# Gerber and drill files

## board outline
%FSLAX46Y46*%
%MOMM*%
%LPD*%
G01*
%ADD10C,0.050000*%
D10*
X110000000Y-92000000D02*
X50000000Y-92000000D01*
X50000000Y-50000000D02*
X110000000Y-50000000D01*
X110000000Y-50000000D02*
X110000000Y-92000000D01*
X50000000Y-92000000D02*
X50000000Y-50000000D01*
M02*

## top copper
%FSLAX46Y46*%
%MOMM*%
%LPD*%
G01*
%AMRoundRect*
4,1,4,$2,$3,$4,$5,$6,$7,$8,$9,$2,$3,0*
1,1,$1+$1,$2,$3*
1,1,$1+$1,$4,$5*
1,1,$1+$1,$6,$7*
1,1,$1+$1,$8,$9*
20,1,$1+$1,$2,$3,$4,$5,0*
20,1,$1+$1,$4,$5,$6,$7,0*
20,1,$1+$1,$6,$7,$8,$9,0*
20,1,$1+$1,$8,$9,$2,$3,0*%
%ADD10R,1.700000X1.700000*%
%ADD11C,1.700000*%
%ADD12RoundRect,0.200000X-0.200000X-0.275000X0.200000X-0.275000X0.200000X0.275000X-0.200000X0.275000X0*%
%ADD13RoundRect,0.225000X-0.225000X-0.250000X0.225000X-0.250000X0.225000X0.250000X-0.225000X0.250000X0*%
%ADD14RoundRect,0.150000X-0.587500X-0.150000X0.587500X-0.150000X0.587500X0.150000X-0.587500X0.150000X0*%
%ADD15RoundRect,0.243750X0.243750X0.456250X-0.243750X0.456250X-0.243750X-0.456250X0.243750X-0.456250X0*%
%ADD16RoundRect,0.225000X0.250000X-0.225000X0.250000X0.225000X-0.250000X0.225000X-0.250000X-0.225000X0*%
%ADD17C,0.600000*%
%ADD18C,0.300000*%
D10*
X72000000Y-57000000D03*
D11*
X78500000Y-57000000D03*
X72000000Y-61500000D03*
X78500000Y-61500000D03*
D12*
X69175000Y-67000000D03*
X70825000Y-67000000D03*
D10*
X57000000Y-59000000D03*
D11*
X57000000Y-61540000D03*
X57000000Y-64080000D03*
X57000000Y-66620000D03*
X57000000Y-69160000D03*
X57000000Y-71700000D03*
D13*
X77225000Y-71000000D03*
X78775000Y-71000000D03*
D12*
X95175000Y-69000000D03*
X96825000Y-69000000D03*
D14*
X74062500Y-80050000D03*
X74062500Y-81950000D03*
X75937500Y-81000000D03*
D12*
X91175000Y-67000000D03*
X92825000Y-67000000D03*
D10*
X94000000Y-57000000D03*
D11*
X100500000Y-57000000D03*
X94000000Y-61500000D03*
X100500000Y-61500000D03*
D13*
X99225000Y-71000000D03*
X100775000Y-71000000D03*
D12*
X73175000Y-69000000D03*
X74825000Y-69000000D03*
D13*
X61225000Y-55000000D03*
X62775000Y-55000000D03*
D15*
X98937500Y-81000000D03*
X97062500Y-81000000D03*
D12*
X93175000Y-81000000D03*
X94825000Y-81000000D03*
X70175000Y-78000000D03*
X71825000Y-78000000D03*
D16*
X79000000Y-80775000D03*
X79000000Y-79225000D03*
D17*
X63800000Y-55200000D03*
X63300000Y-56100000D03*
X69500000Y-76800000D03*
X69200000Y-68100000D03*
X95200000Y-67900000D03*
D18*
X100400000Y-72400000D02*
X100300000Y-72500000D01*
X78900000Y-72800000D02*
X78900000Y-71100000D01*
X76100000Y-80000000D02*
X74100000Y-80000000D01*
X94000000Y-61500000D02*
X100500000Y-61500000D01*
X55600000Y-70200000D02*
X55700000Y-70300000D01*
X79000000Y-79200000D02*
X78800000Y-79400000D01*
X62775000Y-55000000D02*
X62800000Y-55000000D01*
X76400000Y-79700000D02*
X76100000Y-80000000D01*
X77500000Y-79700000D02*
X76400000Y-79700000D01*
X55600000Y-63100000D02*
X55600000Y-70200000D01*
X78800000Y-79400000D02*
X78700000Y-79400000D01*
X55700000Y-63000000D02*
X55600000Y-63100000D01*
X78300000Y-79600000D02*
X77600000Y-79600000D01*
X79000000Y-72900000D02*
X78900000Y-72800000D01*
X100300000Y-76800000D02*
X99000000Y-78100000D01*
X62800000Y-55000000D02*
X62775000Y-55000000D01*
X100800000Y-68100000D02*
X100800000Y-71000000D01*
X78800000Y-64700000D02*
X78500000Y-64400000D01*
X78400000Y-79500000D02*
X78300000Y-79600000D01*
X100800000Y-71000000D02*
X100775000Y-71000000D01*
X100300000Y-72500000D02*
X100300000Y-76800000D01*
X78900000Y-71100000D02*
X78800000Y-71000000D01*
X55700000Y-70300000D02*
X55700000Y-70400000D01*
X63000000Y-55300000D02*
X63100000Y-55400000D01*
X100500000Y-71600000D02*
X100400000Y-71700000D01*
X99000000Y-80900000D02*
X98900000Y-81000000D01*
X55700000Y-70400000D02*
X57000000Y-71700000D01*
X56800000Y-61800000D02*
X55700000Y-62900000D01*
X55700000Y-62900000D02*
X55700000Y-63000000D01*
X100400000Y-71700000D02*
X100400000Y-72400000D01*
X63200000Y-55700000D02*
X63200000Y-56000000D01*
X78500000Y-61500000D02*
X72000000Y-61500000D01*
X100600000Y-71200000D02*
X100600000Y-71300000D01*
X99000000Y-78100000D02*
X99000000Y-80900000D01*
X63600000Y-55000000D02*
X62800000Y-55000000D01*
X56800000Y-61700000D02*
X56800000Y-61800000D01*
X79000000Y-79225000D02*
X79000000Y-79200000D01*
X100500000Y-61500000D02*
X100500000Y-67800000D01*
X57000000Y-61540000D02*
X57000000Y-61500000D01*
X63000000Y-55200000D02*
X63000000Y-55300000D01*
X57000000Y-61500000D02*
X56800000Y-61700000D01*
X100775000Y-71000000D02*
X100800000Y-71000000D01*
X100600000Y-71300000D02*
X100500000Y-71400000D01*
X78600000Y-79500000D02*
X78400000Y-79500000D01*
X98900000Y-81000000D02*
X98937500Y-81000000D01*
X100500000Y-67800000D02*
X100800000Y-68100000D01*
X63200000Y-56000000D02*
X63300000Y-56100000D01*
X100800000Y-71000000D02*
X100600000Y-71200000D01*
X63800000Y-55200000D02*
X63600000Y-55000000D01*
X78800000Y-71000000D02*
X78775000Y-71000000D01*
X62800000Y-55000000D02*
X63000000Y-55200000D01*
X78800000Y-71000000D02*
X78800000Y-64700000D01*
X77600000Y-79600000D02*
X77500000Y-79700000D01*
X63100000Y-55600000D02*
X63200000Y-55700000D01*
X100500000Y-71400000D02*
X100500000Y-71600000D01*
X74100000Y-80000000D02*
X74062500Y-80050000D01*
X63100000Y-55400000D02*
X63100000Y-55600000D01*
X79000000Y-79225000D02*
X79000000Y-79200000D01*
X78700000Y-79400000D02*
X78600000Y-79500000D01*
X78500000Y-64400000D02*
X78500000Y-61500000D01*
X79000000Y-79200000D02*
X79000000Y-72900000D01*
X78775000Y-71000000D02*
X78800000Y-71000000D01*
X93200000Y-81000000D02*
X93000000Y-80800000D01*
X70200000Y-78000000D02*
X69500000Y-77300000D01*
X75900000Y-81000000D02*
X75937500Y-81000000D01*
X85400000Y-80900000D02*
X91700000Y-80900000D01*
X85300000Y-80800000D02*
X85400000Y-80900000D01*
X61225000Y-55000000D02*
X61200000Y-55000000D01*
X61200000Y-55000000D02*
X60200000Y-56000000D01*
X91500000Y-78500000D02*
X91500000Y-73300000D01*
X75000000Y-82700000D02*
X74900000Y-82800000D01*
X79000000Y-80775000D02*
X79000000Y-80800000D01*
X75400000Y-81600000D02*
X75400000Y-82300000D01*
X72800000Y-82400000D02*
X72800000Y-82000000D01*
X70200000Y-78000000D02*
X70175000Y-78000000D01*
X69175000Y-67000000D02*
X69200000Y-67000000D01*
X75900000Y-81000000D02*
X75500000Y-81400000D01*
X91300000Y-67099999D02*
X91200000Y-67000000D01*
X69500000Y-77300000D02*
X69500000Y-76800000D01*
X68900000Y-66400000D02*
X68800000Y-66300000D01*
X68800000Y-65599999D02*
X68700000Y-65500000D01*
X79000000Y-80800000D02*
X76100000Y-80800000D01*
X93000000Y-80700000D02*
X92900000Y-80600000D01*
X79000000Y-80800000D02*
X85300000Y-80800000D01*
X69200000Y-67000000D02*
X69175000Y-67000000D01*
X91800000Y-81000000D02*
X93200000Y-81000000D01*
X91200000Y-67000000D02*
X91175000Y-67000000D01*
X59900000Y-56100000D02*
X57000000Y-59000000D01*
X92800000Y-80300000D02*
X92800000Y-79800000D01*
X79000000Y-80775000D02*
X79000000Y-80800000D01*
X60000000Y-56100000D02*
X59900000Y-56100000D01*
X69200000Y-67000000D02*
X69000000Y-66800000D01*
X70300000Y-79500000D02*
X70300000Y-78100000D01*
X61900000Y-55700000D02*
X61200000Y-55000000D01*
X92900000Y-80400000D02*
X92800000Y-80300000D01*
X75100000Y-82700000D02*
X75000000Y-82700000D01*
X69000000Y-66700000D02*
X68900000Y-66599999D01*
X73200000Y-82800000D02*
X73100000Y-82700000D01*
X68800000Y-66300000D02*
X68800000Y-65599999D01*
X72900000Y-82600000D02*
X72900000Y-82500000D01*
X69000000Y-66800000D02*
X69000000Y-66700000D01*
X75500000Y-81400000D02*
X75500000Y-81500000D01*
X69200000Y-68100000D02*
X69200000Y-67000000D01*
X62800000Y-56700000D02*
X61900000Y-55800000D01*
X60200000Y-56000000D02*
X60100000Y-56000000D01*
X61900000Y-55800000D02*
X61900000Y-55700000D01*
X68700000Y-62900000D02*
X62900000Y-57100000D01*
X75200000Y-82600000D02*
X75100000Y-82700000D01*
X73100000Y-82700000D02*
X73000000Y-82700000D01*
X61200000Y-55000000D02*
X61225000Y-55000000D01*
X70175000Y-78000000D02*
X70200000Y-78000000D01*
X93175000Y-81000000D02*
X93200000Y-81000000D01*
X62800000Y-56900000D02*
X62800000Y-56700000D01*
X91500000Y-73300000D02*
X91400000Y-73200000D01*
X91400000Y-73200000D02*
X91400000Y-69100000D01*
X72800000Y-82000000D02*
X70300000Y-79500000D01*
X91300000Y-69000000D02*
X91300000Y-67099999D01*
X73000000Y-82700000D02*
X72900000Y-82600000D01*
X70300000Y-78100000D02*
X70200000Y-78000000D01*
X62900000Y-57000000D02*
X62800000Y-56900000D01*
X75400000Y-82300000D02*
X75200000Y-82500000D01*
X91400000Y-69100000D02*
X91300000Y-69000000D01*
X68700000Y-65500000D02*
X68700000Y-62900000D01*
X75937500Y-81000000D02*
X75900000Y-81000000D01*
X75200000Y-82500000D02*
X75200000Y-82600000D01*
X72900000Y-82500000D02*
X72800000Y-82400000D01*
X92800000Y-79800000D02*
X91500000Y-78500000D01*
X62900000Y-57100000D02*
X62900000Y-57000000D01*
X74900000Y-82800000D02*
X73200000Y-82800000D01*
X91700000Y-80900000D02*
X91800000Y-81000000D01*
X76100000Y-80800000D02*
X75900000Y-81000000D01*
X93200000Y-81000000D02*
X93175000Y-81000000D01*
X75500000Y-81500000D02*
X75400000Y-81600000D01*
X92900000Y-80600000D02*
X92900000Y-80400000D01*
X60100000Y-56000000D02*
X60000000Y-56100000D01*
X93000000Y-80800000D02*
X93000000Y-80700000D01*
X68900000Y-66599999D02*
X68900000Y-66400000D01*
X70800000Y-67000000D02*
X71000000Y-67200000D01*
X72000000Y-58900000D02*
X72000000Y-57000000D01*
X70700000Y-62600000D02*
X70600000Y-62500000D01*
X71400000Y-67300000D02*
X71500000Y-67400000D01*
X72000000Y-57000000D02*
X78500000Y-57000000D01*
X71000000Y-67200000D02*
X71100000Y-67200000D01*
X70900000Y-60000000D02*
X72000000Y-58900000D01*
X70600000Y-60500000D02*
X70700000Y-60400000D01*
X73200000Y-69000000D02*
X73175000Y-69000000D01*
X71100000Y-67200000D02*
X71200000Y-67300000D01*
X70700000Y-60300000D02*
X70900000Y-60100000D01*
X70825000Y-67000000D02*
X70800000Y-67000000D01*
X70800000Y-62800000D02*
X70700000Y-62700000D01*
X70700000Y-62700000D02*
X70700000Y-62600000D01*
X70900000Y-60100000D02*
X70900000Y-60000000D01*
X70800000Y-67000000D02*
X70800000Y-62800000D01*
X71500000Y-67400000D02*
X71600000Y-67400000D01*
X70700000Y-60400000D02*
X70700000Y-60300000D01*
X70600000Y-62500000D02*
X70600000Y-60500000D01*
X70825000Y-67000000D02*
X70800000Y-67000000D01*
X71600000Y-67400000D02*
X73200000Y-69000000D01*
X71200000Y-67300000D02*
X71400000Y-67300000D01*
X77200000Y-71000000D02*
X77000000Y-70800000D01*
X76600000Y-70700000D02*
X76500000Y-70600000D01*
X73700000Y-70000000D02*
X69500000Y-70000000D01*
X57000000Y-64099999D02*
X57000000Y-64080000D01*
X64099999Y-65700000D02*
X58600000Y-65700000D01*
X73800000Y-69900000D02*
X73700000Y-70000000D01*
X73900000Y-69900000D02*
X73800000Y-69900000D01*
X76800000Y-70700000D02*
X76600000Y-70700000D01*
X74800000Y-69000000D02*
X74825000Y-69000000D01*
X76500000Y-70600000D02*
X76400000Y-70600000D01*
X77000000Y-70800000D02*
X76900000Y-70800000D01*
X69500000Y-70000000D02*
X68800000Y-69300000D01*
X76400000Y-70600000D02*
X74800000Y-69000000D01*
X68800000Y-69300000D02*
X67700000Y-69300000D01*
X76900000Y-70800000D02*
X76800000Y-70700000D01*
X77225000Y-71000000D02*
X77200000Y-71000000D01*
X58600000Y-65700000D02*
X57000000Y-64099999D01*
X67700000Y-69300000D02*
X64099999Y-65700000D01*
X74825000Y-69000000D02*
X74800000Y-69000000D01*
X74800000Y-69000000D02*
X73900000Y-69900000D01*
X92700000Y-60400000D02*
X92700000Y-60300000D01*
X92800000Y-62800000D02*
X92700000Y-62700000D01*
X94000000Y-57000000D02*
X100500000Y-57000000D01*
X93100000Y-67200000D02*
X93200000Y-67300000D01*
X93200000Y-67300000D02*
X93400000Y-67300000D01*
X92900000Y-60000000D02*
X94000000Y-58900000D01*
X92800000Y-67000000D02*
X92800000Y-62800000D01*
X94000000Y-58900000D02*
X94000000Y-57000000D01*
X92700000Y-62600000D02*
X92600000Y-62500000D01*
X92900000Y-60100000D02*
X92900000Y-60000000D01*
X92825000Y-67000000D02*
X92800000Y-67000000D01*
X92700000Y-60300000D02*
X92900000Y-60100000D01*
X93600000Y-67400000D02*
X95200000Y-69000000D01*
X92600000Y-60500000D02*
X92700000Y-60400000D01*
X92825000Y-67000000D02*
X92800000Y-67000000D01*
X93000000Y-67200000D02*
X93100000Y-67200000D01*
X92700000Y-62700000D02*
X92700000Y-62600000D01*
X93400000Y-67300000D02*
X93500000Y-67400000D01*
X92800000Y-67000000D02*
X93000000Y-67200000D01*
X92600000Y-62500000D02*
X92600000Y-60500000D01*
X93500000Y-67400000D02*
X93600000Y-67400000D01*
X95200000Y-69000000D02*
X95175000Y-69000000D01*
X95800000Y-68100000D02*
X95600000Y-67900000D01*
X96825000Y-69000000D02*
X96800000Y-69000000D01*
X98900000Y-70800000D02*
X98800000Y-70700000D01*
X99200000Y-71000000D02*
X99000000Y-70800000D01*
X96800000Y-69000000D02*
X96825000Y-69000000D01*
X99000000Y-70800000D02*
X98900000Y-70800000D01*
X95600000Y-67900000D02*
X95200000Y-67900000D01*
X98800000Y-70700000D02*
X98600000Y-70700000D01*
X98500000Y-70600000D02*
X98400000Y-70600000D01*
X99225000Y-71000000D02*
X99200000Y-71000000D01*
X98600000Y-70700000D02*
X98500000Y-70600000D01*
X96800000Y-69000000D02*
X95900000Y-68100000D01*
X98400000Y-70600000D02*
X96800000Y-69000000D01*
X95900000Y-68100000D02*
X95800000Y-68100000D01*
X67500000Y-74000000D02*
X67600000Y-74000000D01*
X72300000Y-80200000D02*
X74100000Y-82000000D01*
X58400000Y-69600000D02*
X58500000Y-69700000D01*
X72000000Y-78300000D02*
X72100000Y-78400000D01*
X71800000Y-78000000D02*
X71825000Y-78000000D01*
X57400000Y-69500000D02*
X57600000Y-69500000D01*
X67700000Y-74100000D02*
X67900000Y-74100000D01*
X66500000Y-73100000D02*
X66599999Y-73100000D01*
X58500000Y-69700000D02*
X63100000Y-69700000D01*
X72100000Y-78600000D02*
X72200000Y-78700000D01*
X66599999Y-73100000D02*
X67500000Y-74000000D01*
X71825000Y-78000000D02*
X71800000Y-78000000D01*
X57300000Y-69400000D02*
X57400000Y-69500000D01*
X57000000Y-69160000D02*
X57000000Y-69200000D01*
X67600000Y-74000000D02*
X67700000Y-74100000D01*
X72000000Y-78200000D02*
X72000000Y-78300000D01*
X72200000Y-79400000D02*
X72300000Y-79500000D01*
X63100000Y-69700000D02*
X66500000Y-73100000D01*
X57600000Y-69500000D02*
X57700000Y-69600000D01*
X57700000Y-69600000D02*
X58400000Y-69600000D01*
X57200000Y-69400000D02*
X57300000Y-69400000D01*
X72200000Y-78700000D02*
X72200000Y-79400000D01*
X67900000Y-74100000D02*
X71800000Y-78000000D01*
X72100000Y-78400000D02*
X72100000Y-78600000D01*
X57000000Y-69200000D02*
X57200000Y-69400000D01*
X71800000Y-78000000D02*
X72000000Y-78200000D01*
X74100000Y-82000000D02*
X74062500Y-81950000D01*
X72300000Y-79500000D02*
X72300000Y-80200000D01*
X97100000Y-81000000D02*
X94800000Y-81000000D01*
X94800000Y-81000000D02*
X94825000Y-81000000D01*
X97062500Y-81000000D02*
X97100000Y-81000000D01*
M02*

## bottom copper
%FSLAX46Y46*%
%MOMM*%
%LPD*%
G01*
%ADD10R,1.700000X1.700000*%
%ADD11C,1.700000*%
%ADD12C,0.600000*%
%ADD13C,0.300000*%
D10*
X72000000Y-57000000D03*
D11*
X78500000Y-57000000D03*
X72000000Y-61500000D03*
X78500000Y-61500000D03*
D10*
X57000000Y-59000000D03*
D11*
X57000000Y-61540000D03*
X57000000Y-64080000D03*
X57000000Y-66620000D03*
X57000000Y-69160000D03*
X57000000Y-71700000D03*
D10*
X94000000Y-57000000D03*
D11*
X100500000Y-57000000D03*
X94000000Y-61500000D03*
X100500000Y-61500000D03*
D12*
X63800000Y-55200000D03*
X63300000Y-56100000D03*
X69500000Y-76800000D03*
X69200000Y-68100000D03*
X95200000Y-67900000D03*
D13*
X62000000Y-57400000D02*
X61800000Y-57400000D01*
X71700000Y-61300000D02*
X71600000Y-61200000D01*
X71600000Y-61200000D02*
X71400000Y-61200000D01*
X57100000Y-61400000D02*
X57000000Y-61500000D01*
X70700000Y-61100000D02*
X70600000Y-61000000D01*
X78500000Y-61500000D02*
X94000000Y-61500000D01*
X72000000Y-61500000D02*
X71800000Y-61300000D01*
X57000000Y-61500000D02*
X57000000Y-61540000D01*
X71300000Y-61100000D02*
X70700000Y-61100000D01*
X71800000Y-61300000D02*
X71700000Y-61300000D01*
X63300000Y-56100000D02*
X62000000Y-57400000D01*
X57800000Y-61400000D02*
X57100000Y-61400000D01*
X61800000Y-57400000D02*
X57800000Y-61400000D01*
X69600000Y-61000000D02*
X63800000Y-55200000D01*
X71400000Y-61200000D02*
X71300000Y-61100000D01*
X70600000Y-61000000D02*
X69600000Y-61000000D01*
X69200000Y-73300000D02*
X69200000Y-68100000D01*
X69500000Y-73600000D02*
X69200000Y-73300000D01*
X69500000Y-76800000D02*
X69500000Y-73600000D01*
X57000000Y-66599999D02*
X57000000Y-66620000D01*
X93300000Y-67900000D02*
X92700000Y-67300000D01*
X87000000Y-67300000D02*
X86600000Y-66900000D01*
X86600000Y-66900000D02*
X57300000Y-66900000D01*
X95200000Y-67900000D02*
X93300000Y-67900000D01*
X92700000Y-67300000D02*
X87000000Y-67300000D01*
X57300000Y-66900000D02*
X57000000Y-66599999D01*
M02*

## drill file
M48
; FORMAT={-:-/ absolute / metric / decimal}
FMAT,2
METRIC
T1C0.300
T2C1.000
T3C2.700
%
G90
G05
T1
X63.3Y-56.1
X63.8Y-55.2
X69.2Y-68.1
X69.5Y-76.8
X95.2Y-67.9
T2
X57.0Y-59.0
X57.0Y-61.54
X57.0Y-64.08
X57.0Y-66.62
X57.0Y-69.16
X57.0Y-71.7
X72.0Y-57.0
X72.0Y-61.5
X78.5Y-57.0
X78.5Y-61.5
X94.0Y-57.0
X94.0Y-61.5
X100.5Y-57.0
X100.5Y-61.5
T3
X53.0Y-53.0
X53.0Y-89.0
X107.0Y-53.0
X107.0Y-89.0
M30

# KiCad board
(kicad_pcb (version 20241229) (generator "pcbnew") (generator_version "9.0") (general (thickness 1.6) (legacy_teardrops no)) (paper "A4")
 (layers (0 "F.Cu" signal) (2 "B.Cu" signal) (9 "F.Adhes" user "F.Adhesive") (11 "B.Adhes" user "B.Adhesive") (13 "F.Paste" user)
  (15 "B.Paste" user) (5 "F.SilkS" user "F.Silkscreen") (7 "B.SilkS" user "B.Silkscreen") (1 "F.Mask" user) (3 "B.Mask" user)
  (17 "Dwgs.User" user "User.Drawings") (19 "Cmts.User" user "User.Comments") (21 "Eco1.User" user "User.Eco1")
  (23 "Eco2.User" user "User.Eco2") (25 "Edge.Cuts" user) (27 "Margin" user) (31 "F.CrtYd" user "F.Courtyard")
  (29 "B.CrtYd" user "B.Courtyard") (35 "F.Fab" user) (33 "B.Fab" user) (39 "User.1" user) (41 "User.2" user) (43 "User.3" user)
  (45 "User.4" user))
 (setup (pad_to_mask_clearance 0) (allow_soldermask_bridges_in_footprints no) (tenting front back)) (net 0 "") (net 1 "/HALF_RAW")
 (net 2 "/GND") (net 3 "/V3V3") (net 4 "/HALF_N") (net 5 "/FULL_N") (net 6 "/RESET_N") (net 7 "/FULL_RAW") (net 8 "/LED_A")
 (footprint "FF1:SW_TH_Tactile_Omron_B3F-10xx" (layer "F.Cu") (at 72 57)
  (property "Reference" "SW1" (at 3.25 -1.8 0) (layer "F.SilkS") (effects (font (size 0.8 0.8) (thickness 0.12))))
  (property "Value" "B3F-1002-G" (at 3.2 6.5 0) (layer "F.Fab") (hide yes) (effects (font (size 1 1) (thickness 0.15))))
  (pad "1" thru_hole rect (at 0 0) (size 1.7 1.7) (drill 1) (layers "*.Cu" "*.Mask") (remove_unused_layers no) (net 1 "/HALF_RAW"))
  (pad "1" thru_hole circle (at 6.5 0) (size 1.7 1.7) (drill 1) (layers "*.Cu" "*.Mask") (remove_unused_layers no) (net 1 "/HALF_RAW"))
  (pad "2" thru_hole circle (at 0 4.5) (size 1.7 1.7) (drill 1) (layers "*.Cu" "*.Mask") (remove_unused_layers no) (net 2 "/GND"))
  (pad "2" thru_hole circle (at 6.5 4.5) (size 1.7 1.7) (drill 1) (layers "*.Cu" "*.Mask") (remove_unused_layers no) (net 2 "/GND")))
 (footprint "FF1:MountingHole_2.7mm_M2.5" (layer "F.Cu") (at 53 53)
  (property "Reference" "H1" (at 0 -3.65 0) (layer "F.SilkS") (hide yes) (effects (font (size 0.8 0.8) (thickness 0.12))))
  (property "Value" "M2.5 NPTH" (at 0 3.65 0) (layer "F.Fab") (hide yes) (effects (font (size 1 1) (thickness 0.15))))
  (pad "" np_thru_hole circle (at 0 0) (size 2.7 2.7) (drill 2.7) (layers "*.Cu" "*.Mask")))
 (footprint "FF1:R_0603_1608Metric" (layer "F.Cu") (at 70 67)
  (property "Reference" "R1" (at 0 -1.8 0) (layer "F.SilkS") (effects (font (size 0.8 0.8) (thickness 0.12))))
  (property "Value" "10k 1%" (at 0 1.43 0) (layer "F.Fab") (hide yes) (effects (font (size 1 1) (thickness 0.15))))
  (pad "1" smd roundrect (at -0.825 0) (size 0.8 0.95) (layers "F.Cu" "F.Mask" "F.Paste") (roundrect_rratio 0.25) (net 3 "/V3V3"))
  (pad "2" smd roundrect (at 0.825 0) (size 0.8 0.95) (layers "F.Cu" "F.Mask" "F.Paste") (roundrect_rratio 0.25) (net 1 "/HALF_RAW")))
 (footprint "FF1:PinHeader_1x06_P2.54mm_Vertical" (layer "F.Cu") (at 57 59)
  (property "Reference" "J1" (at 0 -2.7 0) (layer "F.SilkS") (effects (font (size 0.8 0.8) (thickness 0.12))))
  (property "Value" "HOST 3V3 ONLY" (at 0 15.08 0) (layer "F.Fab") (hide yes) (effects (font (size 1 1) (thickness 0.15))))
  (pad "1" thru_hole rect (at 0 0) (size 1.7 1.7) (drill 1) (layers "*.Cu" "*.Mask") (remove_unused_layers no) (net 3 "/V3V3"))
  (pad "2" thru_hole circle (at 0 2.54) (size 1.7 1.7) (drill 1) (layers "*.Cu" "*.Mask") (remove_unused_layers no) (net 2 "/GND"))
  (pad "3" thru_hole circle (at 0 5.08) (size 1.7 1.7) (drill 1) (layers "*.Cu" "*.Mask") (remove_unused_layers no) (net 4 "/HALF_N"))
  (pad "4" thru_hole circle (at 0 7.62) (size 1.7 1.7) (drill 1) (layers "*.Cu" "*.Mask") (remove_unused_layers no) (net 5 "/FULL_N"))
  (pad "5" thru_hole circle (at 0 10.16) (size 1.7 1.7) (drill 1) (layers "*.Cu" "*.Mask") (remove_unused_layers no) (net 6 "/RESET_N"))
  (pad "6" thru_hole circle (at 0 12.7) (size 1.7 1.7) (drill 1) (layers "*.Cu" "*.Mask") (remove_unused_layers no) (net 2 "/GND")))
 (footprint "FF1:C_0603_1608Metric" (layer "F.Cu") (at 78 71)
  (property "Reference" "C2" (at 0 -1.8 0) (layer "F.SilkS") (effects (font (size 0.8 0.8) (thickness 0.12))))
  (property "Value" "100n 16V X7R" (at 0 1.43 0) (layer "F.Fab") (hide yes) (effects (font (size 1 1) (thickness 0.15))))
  (pad "1" smd roundrect (at -0.775 0) (size 0.9 0.95) (layers "F.Cu" "F.Mask" "F.Paste") (roundrect_rratio 0.25) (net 4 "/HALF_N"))
  (pad "2" smd roundrect (at 0.775 0) (size 0.9 0.95) (layers "F.Cu" "F.Mask" "F.Paste") (roundrect_rratio 0.25) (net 2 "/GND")))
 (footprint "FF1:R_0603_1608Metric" (layer "F.Cu") (at 96 69)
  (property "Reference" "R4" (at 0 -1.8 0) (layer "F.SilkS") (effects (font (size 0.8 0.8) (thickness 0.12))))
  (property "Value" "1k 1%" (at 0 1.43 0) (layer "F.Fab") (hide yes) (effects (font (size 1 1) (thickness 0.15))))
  (pad "1" smd roundrect (at -0.825 0) (size 0.8 0.95) (layers "F.Cu" "F.Mask" "F.Paste") (roundrect_rratio 0.25) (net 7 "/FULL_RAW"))
  (pad "2" smd roundrect (at 0.825 0) (size 0.8 0.95) (layers "F.Cu" "F.Mask" "F.Paste") (roundrect_rratio 0.25) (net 5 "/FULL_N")))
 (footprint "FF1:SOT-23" (layer "F.Cu") (at 75 81)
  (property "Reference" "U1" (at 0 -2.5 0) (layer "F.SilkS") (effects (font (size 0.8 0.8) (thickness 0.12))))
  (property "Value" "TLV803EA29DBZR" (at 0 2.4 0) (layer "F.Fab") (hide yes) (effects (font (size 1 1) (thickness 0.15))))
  (pad "1" smd roundrect (at -0.9375 -0.95) (size 1.475 0.6) (layers "F.Cu" "F.Mask" "F.Paste") (roundrect_rratio 0.25) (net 2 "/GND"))
  (pad "2" smd roundrect (at -0.9375 0.95) (size 1.475 0.6) (layers "F.Cu" "F.Mask" "F.Paste") (roundrect_rratio 0.25) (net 6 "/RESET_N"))
  (pad "3" smd roundrect (at 0.9375 0) (size 1.475 0.6) (layers "F.Cu" "F.Mask" "F.Paste") (roundrect_rratio 0.25) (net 3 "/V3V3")))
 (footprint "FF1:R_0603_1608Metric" (layer "F.Cu") (at 92 67)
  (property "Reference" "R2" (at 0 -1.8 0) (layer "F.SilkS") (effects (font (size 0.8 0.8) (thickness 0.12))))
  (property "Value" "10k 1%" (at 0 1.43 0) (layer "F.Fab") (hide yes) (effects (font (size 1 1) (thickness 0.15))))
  (pad "1" smd roundrect (at -0.825 0) (size 0.8 0.95) (layers "F.Cu" "F.Mask" "F.Paste") (roundrect_rratio 0.25) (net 3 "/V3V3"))
  (pad "2" smd roundrect (at 0.825 0) (size 0.8 0.95) (layers "F.Cu" "F.Mask" "F.Paste") (roundrect_rratio 0.25) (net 7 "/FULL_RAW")))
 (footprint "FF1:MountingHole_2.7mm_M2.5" (layer "F.Cu") (at 107 53)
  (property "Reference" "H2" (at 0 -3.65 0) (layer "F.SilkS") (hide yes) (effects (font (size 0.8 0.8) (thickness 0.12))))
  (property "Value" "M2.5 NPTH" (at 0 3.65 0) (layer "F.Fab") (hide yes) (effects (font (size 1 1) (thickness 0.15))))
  (pad "" np_thru_hole circle (at 0 0) (size 2.7 2.7) (drill 2.7) (layers "*.Cu" "*.Mask")))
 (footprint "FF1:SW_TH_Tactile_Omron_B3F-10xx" (layer "F.Cu") (at 94 57)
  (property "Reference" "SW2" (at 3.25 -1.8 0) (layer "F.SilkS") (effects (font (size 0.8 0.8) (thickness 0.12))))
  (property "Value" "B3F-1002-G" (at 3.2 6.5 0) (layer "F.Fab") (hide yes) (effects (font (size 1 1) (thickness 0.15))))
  (pad "1" thru_hole rect (at 0 0) (size 1.7 1.7) (drill 1) (layers "*.Cu" "*.Mask") (remove_unused_layers no) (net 7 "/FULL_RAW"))
  (pad "1" thru_hole circle (at 6.5 0) (size 1.7 1.7) (drill 1) (layers "*.Cu" "*.Mask") (remove_unused_layers no) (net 7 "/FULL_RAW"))
  (pad "2" thru_hole circle (at 0 4.5) (size 1.7 1.7) (drill 1) (layers "*.Cu" "*.Mask") (remove_unused_layers no) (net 2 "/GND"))
  (pad "2" thru_hole circle (at 6.5 4.5) (size 1.7 1.7) (drill 1) (layers "*.Cu" "*.Mask") (remove_unused_layers no) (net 2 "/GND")))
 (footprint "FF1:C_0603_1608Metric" (layer "F.Cu") (at 100 71)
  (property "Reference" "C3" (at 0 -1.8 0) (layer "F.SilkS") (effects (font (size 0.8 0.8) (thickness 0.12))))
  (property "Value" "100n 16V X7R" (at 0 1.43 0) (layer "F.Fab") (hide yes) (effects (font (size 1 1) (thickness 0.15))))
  (pad "1" smd roundrect (at -0.775 0) (size 0.9 0.95) (layers "F.Cu" "F.Mask" "F.Paste") (roundrect_rratio 0.25) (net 5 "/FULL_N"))
  (pad "2" smd roundrect (at 0.775 0) (size 0.9 0.95) (layers "F.Cu" "F.Mask" "F.Paste") (roundrect_rratio 0.25) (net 2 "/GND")))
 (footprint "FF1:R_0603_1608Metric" (layer "F.Cu") (at 74 69)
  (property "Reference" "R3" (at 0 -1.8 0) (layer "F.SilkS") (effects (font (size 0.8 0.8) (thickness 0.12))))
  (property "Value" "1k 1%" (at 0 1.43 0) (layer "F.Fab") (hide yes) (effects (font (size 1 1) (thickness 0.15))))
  (pad "1" smd roundrect (at -0.825 0) (size 0.8 0.95) (layers "F.Cu" "F.Mask" "F.Paste") (roundrect_rratio 0.25) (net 1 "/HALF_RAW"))
  (pad "2" smd roundrect (at 0.825 0) (size 0.8 0.95) (layers "F.Cu" "F.Mask" "F.Paste") (roundrect_rratio 0.25) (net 4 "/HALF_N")))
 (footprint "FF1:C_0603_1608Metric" (layer "F.Cu") (at 62 55)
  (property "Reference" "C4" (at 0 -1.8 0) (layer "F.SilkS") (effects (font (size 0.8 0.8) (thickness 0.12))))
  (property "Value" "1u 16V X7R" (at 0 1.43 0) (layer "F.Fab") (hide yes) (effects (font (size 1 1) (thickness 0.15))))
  (pad "1" smd roundrect (at -0.775 0) (size 0.9 0.95) (layers "F.Cu" "F.Mask" "F.Paste") (roundrect_rratio 0.25) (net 3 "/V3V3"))
  (pad "2" smd roundrect (at 0.775 0) (size 0.9 0.95) (layers "F.Cu" "F.Mask" "F.Paste") (roundrect_rratio 0.25) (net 2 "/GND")))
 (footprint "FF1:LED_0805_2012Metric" (layer "F.Cu") (at 98 81 180)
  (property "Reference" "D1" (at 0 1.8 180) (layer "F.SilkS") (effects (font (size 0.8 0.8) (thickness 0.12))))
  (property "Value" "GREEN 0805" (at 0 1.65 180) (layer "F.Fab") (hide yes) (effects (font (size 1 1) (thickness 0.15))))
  (pad "1" smd roundrect (at -0.9375 0 180) (size 0.975 1.4) (layers "F.Cu" "F.Mask" "F.Paste") (roundrect_rratio 0.25) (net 2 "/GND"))
  (pad "2" smd roundrect (at 0.9375 0 180) (size 0.975 1.4) (layers "F.Cu" "F.Mask" "F.Paste") (roundrect_rratio 0.25) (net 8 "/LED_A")))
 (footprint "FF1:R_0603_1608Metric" (layer "F.Cu") (at 94 81)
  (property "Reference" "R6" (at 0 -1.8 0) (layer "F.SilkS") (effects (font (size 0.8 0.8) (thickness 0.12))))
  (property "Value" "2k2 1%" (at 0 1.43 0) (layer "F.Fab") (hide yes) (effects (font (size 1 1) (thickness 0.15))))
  (pad "1" smd roundrect (at -0.825 0) (size 0.8 0.95) (layers "F.Cu" "F.Mask" "F.Paste") (roundrect_rratio 0.25) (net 3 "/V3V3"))
  (pad "2" smd roundrect (at 0.825 0) (size 0.8 0.95) (layers "F.Cu" "F.Mask" "F.Paste") (roundrect_rratio 0.25) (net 8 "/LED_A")))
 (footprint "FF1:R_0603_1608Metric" (layer "F.Cu") (at 71 78)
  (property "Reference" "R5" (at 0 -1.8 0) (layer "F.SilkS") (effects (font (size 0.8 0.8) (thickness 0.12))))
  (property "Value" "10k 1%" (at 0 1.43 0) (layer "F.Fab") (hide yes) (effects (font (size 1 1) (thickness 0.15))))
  (pad "1" smd roundrect (at -0.825 0) (size 0.8 0.95) (layers "F.Cu" "F.Mask" "F.Paste") (roundrect_rratio 0.25) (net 3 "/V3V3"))
  (pad "2" smd roundrect (at 0.825 0) (size 0.8 0.95) (layers "F.Cu" "F.Mask" "F.Paste") (roundrect_rratio 0.25) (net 6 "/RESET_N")))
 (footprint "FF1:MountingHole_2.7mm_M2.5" (layer "F.Cu") (at 53 89)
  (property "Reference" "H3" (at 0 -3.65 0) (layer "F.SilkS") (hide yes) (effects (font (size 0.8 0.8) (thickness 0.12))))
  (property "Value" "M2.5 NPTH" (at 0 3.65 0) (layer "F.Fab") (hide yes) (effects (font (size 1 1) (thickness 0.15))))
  (pad "" np_thru_hole circle (at 0 0) (size 2.7 2.7) (drill 2.7) (layers "*.Cu" "*.Mask")))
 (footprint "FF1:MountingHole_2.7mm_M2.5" (layer "F.Cu") (at 107 89)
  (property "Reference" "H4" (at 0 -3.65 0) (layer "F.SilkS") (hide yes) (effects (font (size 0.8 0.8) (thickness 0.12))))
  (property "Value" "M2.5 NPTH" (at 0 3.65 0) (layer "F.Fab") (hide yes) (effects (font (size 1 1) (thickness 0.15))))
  (pad "" np_thru_hole circle (at 0 0) (size 2.7 2.7) (drill 2.7) (layers "*.Cu" "*.Mask")))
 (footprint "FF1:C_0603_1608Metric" (layer "F.Cu") (at 79 80 90)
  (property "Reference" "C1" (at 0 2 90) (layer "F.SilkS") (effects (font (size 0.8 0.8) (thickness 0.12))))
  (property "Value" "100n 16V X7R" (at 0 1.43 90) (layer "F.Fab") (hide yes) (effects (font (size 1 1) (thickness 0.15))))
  (pad "1" smd roundrect (at -0.775 0 90) (size 0.9 0.95) (layers "F.Cu" "F.Mask" "F.Paste") (roundrect_rratio 0.25) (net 3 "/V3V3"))
  (pad "2" smd roundrect (at 0.775 0 90) (size 0.9 0.95) (layers "F.Cu" "F.Mask" "F.Paste") (roundrect_rratio 0.25) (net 2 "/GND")))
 (gr_line (start 110 92) (end 50 92) (stroke (width 0.05) (type default)) (layer "Edge.Cuts"))
 (gr_line (start 50 50) (end 110 50) (stroke (width 0.05) (type default)) (layer "Edge.Cuts"))
 (gr_line (start 110 50) (end 110 92) (stroke (width 0.05) (type default)) (layer "Edge.Cuts"))
 (gr_line (start 50 92) (end 50 50) (stroke (width 0.05) (type default)) (layer "Edge.Cuts"))
 (segment (start 100.4 72.4) (end 100.3 72.5) (width 0.3) (layer "F.Cu") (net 2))
 (segment (start 78.9 72.8) (end 78.9 71.1) (width 0.3) (layer "F.Cu") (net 2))
 (segment (start 76.1 80) (end 74.1 80) (width 0.3) (layer "F.Cu") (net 2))
 (segment (start 94 61.5) (end 100.5 61.5) (width 0.3) (layer "F.Cu") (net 2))
 (segment (start 55.6 70.2) (end 55.7 70.3) (width 0.3) (layer "F.Cu") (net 2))
 (segment (start 79 79.2) (end 78.8 79.4) (width 0.3) (layer "F.Cu") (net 2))
 (segment (start 62.775 55) (end 62.8 55) (width 0.3) (layer "F.Cu") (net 2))
 (segment (start 76.4 79.7) (end 76.1 80) (width 0.3) (layer "F.Cu") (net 2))
 (segment (start 77.5 79.7) (end 76.4 79.7) (width 0.3) (layer "F.Cu") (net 2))
 (segment (start 55.6 63.1) (end 55.6 70.2) (width 0.3) (layer "F.Cu") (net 2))
 (segment (start 78.8 79.4) (end 78.7 79.4) (width 0.3) (layer "F.Cu") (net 2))
 (segment (start 55.7 63) (end 55.6 63.1) (width 0.3) (layer "F.Cu") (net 2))
 (segment (start 78.3 79.6) (end 77.6 79.6) (width 0.3) (layer "F.Cu") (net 2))
 (segment (start 79 72.9) (end 78.9 72.8) (width 0.3) (layer "F.Cu") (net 2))
 (segment (start 100.3 76.8) (end 99 78.1) (width 0.3) (layer "F.Cu") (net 2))
 (segment (start 62.8 55) (end 62.775 55) (width 0.3) (layer "F.Cu") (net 2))
 (segment (start 100.8 68.1) (end 100.8 71) (width 0.3) (layer "F.Cu") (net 2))
 (segment (start 78.8 64.7) (end 78.5 64.4) (width 0.3) (layer "F.Cu") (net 2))
 (segment (start 78.4 79.5) (end 78.3 79.6) (width 0.3) (layer "F.Cu") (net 2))
 (segment (start 100.8 71) (end 100.775 71) (width 0.3) (layer "F.Cu") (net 2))
 (segment (start 100.3 72.5) (end 100.3 76.8) (width 0.3) (layer "F.Cu") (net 2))
 (segment (start 78.9 71.1) (end 78.8 71) (width 0.3) (layer "F.Cu") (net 2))
 (segment (start 55.7 70.3) (end 55.7 70.4) (width 0.3) (layer "F.Cu") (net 2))
 (segment (start 63 55.3) (end 63.1 55.4) (width 0.3) (layer "F.Cu") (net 2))
 (segment (start 100.5 71.6) (end 100.4 71.7) (width 0.3) (layer "F.Cu") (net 2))
 (segment (start 99 80.9) (end 98.9 81) (width 0.3) (layer "F.Cu") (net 2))
 (segment (start 55.7 70.4) (end 57 71.7) (width 0.3) (layer "F.Cu") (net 2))
 (segment (start 56.8 61.8) (end 55.7 62.9) (width 0.3) (layer "F.Cu") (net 2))
 (segment (start 55.7 62.9) (end 55.7 63) (width 0.3) (layer "F.Cu") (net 2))
 (segment (start 100.4 71.7) (end 100.4 72.4) (width 0.3) (layer "F.Cu") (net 2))
 (segment (start 63.2 55.7) (end 63.2 56) (width 0.3) (layer "F.Cu") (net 2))
 (segment (start 78.5 61.5) (end 72 61.5) (width 0.3) (layer "F.Cu") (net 2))
 (segment (start 100.6 71.2) (end 100.6 71.3) (width 0.3) (layer "F.Cu") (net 2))
 (segment (start 99 78.1) (end 99 80.9) (width 0.3) (layer "F.Cu") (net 2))
 (segment (start 63.6 55) (end 62.8 55) (width 0.3) (layer "F.Cu") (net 2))
 (segment (start 56.8 61.7) (end 56.8 61.8) (width 0.3) (layer "F.Cu") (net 2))
 (segment (start 79 79.225) (end 79 79.2) (width 0.3) (layer "F.Cu") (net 2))
 (segment (start 100.5 61.5) (end 100.5 67.8) (width 0.3) (layer "F.Cu") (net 2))
 (segment (start 57 61.54) (end 57 61.5) (width 0.3) (layer "F.Cu") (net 2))
 (segment (start 63 55.2) (end 63 55.3) (width 0.3) (layer "F.Cu") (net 2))
 (segment (start 57 61.5) (end 56.8 61.7) (width 0.3) (layer "F.Cu") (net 2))
 (segment (start 100.775 71) (end 100.8 71) (width 0.3) (layer "F.Cu") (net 2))
 (segment (start 100.6 71.3) (end 100.5 71.4) (width 0.3) (layer "F.Cu") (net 2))
 (segment (start 78.6 79.5) (end 78.4 79.5) (width 0.3) (layer "F.Cu") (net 2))
 (segment (start 98.9 81) (end 98.9375 81) (width 0.3) (layer "F.Cu") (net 2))
 (segment (start 100.5 67.8) (end 100.8 68.1) (width 0.3) (layer "F.Cu") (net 2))
 (segment (start 63.2 56) (end 63.3 56.1) (width 0.3) (layer "F.Cu") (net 2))
 (segment (start 100.8 71) (end 100.6 71.2) (width 0.3) (layer "F.Cu") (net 2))
 (segment (start 63.8 55.2) (end 63.6 55) (width 0.3) (layer "F.Cu") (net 2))
 (segment (start 78.8 71) (end 78.775 71) (width 0.3) (layer "F.Cu") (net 2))
 (segment (start 62.8 55) (end 63 55.2) (width 0.3) (layer "F.Cu") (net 2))
 (segment (start 78.8 71) (end 78.8 64.7) (width 0.3) (layer "F.Cu") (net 2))
 (segment (start 77.6 79.6) (end 77.5 79.7) (width 0.3) (layer "F.Cu") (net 2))
 (segment (start 63.1 55.6) (end 63.2 55.7) (width 0.3) (layer "F.Cu") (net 2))
 (segment (start 100.5 71.4) (end 100.5 71.6) (width 0.3) (layer "F.Cu") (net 2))
 (segment (start 74.1 80) (end 74.0625 80.05) (width 0.3) (layer "F.Cu") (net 2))
 (segment (start 63.1 55.4) (end 63.1 55.6) (width 0.3) (layer "F.Cu") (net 2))
 (segment (start 79 79.225) (end 79 79.2) (width 0.3) (layer "F.Cu") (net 2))
 (segment (start 78.7 79.4) (end 78.6 79.5) (width 0.3) (layer "F.Cu") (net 2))
 (segment (start 78.5 64.4) (end 78.5 61.5) (width 0.3) (layer "F.Cu") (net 2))
 (segment (start 79 79.2) (end 79 72.9) (width 0.3) (layer "F.Cu") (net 2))
 (segment (start 78.775 71) (end 78.8 71) (width 0.3) (layer "F.Cu") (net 2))
 (via (at 63.8 55.2) (size 0.6) (drill 0.3) (layers "F.Cu" "B.Cu") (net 2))
 (via (at 63.3 56.1) (size 0.6) (drill 0.3) (layers "F.Cu" "B.Cu") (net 2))
 (segment (start 62 57.4) (end 61.8 57.4) (width 0.3) (layer "B.Cu") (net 2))
 (segment (start 71.7 61.3) (end 71.6 61.2) (width 0.3) (layer "B.Cu") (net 2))
 (segment (start 71.6 61.2) (end 71.4 61.2) (width 0.3) (layer "B.Cu") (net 2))
 (segment (start 57.1 61.4) (end 57 61.5) (width 0.3) (layer "B.Cu") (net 2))
 (segment (start 70.7 61.1) (end 70.6 61) (width 0.3) (layer "B.Cu") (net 2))
 (segment (start 78.5 61.5) (end 94 61.5) (width 0.3) (layer "B.Cu") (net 2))
 (segment (start 72 61.5) (end 71.8 61.3) (width 0.3) (layer "B.Cu") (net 2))
 (segment (start 57 61.5) (end 57 61.54) (width 0.3) (layer "B.Cu") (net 2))
 (segment (start 71.3 61.1) (end 70.7 61.1) (width 0.3) (layer "B.Cu") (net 2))
 (segment (start 71.8 61.3) (end 71.7 61.3) (width 0.3) (layer "B.Cu") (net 2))
 (segment (start 63.3 56.1) (end 62 57.4) (width 0.3) (layer "B.Cu") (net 2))
 (segment (start 57.8 61.4) (end 57.1 61.4) (width 0.3) (layer "B.Cu") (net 2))
 (segment (start 61.8 57.4) (end 57.8 61.4) (width 0.3) (layer "B.Cu") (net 2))
 (segment (start 69.6 61) (end 63.8 55.2) (width 0.3) (layer "B.Cu") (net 2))
 (segment (start 71.4 61.2) (end 71.3 61.1) (width 0.3) (layer "B.Cu") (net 2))
 (segment (start 70.6 61) (end 69.6 61) (width 0.3) (layer "B.Cu") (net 2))
 (segment (start 93.2 81) (end 93 80.8) (width 0.3) (layer "F.Cu") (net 3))
 (segment (start 70.2 78) (end 69.5 77.3) (width 0.3) (layer "F.Cu") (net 3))
 (segment (start 75.9 81) (end 75.9375 81) (width 0.3) (layer "F.Cu") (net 3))
 (segment (start 85.4 80.9) (end 91.7 80.9) (width 0.3) (layer "F.Cu") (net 3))
 (segment (start 85.3 80.8) (end 85.4 80.9) (width 0.3) (layer "F.Cu") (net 3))
 (segment (start 61.225 55) (end 61.2 55) (width 0.3) (layer "F.Cu") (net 3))
 (segment (start 61.2 55) (end 60.2 56) (width 0.3) (layer "F.Cu") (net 3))
 (segment (start 91.5 78.5) (end 91.5 73.3) (width 0.3) (layer "F.Cu") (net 3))
 (segment (start 75 82.7) (end 74.9 82.8) (width 0.3) (layer "F.Cu") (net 3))
 (segment (start 79 80.775) (end 79 80.8) (width 0.3) (layer "F.Cu") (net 3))
 (segment (start 75.4 81.6) (end 75.4 82.3) (width 0.3) (layer "F.Cu") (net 3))
 (segment (start 72.8 82.4) (end 72.8 82) (width 0.3) (layer "F.Cu") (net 3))
 (segment (start 70.2 78) (end 70.175 78) (width 0.3) (layer "F.Cu") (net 3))
 (segment (start 69.175 67) (end 69.2 67) (width 0.3) (layer "F.Cu") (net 3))
 (segment (start 75.9 81) (end 75.5 81.4) (width 0.3) (layer "F.Cu") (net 3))
 (segment (start 91.3 67.099999) (end 91.2 67) (width 0.3) (layer "F.Cu") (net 3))
 (segment (start 69.5 77.3) (end 69.5 76.8) (width 0.3) (layer "F.Cu") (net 3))
 (segment (start 68.9 66.4) (end 68.8 66.3) (width 0.3) (layer "F.Cu") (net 3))
 (segment (start 68.8 65.599999) (end 68.7 65.5) (width 0.3) (layer "F.Cu") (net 3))
 (segment (start 79 80.8) (end 76.1 80.8) (width 0.3) (layer "F.Cu") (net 3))
 (segment (start 93 80.7) (end 92.9 80.6) (width 0.3) (layer "F.Cu") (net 3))
 (segment (start 79 80.8) (end 85.3 80.8) (width 0.3) (layer "F.Cu") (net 3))
 (segment (start 69.2 67) (end 69.175 67) (width 0.3) (layer "F.Cu") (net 3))
 (segment (start 91.8 81) (end 93.2 81) (width 0.3) (layer "F.Cu") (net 3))
 (segment (start 91.2 67) (end 91.175 67) (width 0.3) (layer "F.Cu") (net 3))
 (segment (start 59.9 56.1) (end 57 59) (width 0.3) (layer "F.Cu") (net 3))
 (segment (start 92.8 80.3) (end 92.8 79.8) (width 0.3) (layer "F.Cu") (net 3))
 (segment (start 79 80.775) (end 79 80.8) (width 0.3) (layer "F.Cu") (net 3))
 (segment (start 60 56.1) (end 59.9 56.1) (width 0.3) (layer "F.Cu") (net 3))
 (segment (start 69.2 67) (end 69 66.8) (width 0.3) (layer "F.Cu") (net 3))
 (segment (start 70.3 79.5) (end 70.3 78.1) (width 0.3) (layer "F.Cu") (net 3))
 (segment (start 61.9 55.7) (end 61.2 55) (width 0.3) (layer "F.Cu") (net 3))
 (segment (start 92.9 80.4) (end 92.8 80.3) (width 0.3) (layer "F.Cu") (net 3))
 (segment (start 75.1 82.7) (end 75 82.7) (width 0.3) (layer "F.Cu") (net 3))
 (segment (start 69 66.7) (end 68.9 66.599999) (width 0.3) (layer "F.Cu") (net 3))
 (segment (start 73.2 82.8) (end 73.1 82.7) (width 0.3) (layer "F.Cu") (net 3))
 (segment (start 68.8 66.3) (end 68.8 65.599999) (width 0.3) (layer "F.Cu") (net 3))
 (segment (start 72.9 82.6) (end 72.9 82.5) (width 0.3) (layer "F.Cu") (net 3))
 (segment (start 69 66.8) (end 69 66.7) (width 0.3) (layer "F.Cu") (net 3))
 (segment (start 75.5 81.4) (end 75.5 81.5) (width 0.3) (layer "F.Cu") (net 3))
 (segment (start 69.2 68.1) (end 69.2 67) (width 0.3) (layer "F.Cu") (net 3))
 (segment (start 62.8 56.7) (end 61.9 55.8) (width 0.3) (layer "F.Cu") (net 3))
 (segment (start 60.2 56) (end 60.1 56) (width 0.3) (layer "F.Cu") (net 3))
 (segment (start 61.9 55.8) (end 61.9 55.7) (width 0.3) (layer "F.Cu") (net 3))
 (segment (start 68.7 62.9) (end 62.9 57.1) (width 0.3) (layer "F.Cu") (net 3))
 (segment (start 75.2 82.6) (end 75.1 82.7) (width 0.3) (layer "F.Cu") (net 3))
 (segment (start 73.1 82.7) (end 73 82.7) (width 0.3) (layer "F.Cu") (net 3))
 (segment (start 61.2 55) (end 61.225 55) (width 0.3) (layer "F.Cu") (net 3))
 (segment (start 70.175 78) (end 70.2 78) (width 0.3) (layer "F.Cu") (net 3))
 (segment (start 93.175 81) (end 93.2 81) (width 0.3) (layer "F.Cu") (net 3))
 (segment (start 62.8 56.9) (end 62.8 56.7) (width 0.3) (layer "F.Cu") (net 3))
 (segment (start 91.5 73.3) (end 91.4 73.2) (width 0.3) (layer "F.Cu") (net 3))
 (segment (start 91.4 73.2) (end 91.4 69.1) (width 0.3) (layer "F.Cu") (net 3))
 (segment (start 72.8 82) (end 70.3 79.5) (width 0.3) (layer "F.Cu") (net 3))
 (segment (start 91.3 69) (end 91.3 67.099999) (width 0.3) (layer "F.Cu") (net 3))
 (segment (start 73 82.7) (end 72.9 82.6) (width 0.3) (layer "F.Cu") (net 3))
 (segment (start 70.3 78.1) (end 70.2 78) (width 0.3) (layer "F.Cu") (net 3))
 (segment (start 62.9 57) (end 62.8 56.9) (width 0.3) (layer "F.Cu") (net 3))
 (segment (start 75.4 82.3) (end 75.2 82.5) (width 0.3) (layer "F.Cu") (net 3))
 (segment (start 91.4 69.1) (end 91.3 69) (width 0.3) (layer "F.Cu") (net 3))
 (segment (start 68.7 65.5) (end 68.7 62.9) (width 0.3) (layer "F.Cu") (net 3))
 (segment (start 75.9375 81) (end 75.9 81) (width 0.3) (layer "F.Cu") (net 3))
 (segment (start 75.2 82.5) (end 75.2 82.6) (width 0.3) (layer "F.Cu") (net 3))
 (segment (start 72.9 82.5) (end 72.8 82.4) (width 0.3) (layer "F.Cu") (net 3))
 (segment (start 92.8 79.8) (end 91.5 78.5) (width 0.3) (layer "F.Cu") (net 3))
 (segment (start 62.9 57.1) (end 62.9 57) (width 0.3) (layer "F.Cu") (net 3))
 (segment (start 74.9 82.8) (end 73.2 82.8) (width 0.3) (layer "F.Cu") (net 3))
 (segment (start 91.7 80.9) (end 91.8 81) (width 0.3) (layer "F.Cu") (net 3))
 (segment (start 76.1 80.8) (end 75.9 81) (width 0.3) (layer "F.Cu") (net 3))
 (segment (start 93.2 81) (end 93.175 81) (width 0.3) (layer "F.Cu") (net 3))
 (segment (start 75.5 81.5) (end 75.4 81.6) (width 0.3) (layer "F.Cu") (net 3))
 (segment (start 92.9 80.6) (end 92.9 80.4) (width 0.3) (layer "F.Cu") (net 3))
 (segment (start 60.1 56) (end 60 56.1) (width 0.3) (layer "F.Cu") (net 3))
 (segment (start 93 80.8) (end 93 80.7) (width 0.3) (layer "F.Cu") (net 3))
 (segment (start 68.9 66.599999) (end 68.9 66.4) (width 0.3) (layer "F.Cu") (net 3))
 (via (at 69.5 76.8) (size 0.6) (drill 0.3) (layers "F.Cu" "B.Cu") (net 3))
 (via (at 69.2 68.1) (size 0.6) (drill 0.3) (layers "F.Cu" "B.Cu") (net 3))
 (segment (start 69.2 73.3) (end 69.2 68.1) (width 0.3) (layer "B.Cu") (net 3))
 (segment (start 69.5 73.6) (end 69.2 73.3) (width 0.3) (layer "B.Cu") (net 3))
 (segment (start 69.5 76.8) (end 69.5 73.6) (width 0.3) (layer "B.Cu") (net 3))
 (segment (start 70.8 67) (end 71 67.2) (width 0.3) (layer "F.Cu") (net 1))
 (segment (start 72 58.9) (end 72 57) (width 0.3) (layer "F.Cu") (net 1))
 (segment (start 70.7 62.6) (end 70.6 62.5) (width 0.3) (layer "F.Cu") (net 1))
 (segment (start 71.4 67.3) (end 71.5 67.4) (width 0.3) (layer "F.Cu") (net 1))
 (segment (start 72 57) (end 78.5 57) (width 0.3) (layer "F.Cu") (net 1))
 (segment (start 71 67.2) (end 71.1 67.2) (width 0.3) (layer "F.Cu") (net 1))
 (segment (start 70.9 60) (end 72 58.9) (width 0.3) (layer "F.Cu") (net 1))
 (segment (start 70.6 60.5) (end 70.7 60.4) (width 0.3) (layer "F.Cu") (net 1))
 (segment (start 73.2 69) (end 73.175 69) (width 0.3) (layer "F.Cu") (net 1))
 (segment (start 71.1 67.2) (end 71.2 67.3) (width 0.3) (layer "F.Cu") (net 1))
 (segment (start 70.7 60.3) (end 70.9 60.1) (width 0.3) (layer "F.Cu") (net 1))
 (segment (start 70.825 67) (end 70.8 67) (width 0.3) (layer "F.Cu") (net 1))
 (segment (start 70.8 62.8) (end 70.7 62.7) (width 0.3) (layer "F.Cu") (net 1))
 (segment (start 70.7 62.7) (end 70.7 62.6) (width 0.3) (layer "F.Cu") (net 1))
 (segment (start 70.9 60.1) (end 70.9 60) (width 0.3) (layer "F.Cu") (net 1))
 (segment (start 70.8 67) (end 70.8 62.8) (width 0.3) (layer "F.Cu") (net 1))
 (segment (start 71.5 67.4) (end 71.6 67.4) (width 0.3) (layer "F.Cu") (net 1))
 (segment (start 70.7 60.4) (end 70.7 60.3) (width 0.3) (layer "F.Cu") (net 1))
 (segment (start 70.6 62.5) (end 70.6 60.5) (width 0.3) (layer "F.Cu") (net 1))
 (segment (start 70.825 67) (end 70.8 67) (width 0.3) (layer "F.Cu") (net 1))
 (segment (start 71.6 67.4) (end 73.2 69) (width 0.3) (layer "F.Cu") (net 1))
 (segment (start 71.2 67.3) (end 71.4 67.3) (width 0.3) (layer "F.Cu") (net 1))
 (segment (start 77.2 71) (end 77 70.8) (width 0.3) (layer "F.Cu") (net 4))
 (segment (start 76.6 70.7) (end 76.5 70.6) (width 0.3) (layer "F.Cu") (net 4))
 (segment (start 73.7 70) (end 69.5 70) (width 0.3) (layer "F.Cu") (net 4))
 (segment (start 57 64.099999) (end 57 64.08) (width 0.3) (layer "F.Cu") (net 4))
 (segment (start 64.099999 65.7) (end 58.6 65.7) (width 0.3) (layer "F.Cu") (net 4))
 (segment (start 73.8 69.9) (end 73.7 70) (width 0.3) (layer "F.Cu") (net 4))
 (segment (start 73.9 69.9) (end 73.8 69.9) (width 0.3) (layer "F.Cu") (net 4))
 (segment (start 76.8 70.7) (end 76.6 70.7) (width 0.3) (layer "F.Cu") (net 4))
 (segment (start 74.8 69) (end 74.825 69) (width 0.3) (layer "F.Cu") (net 4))
 (segment (start 76.5 70.6) (end 76.4 70.6) (width 0.3) (layer "F.Cu") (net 4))
 (segment (start 77 70.8) (end 76.9 70.8) (width 0.3) (layer "F.Cu") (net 4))
 (segment (start 69.5 70) (end 68.8 69.3) (width 0.3) (layer "F.Cu") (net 4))
 (segment (start 76.4 70.6) (end 74.8 69) (width 0.3) (layer "F.Cu") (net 4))
 (segment (start 68.8 69.3) (end 67.7 69.3) (width 0.3) (layer "F.Cu") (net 4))
 (segment (start 76.9 70.8) (end 76.8 70.7) (width 0.3) (layer "F.Cu") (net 4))
 (segment (start 77.225 71) (end 77.2 71) (width 0.3) (layer "F.Cu") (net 4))
 (segment (start 58.6 65.7) (end 57 64.099999) (width 0.3) (layer "F.Cu") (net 4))
 (segment (start 67.7 69.3) (end 64.099999 65.7) (width 0.3) (layer "F.Cu") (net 4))
 (segment (start 74.825 69) (end 74.8 69) (width 0.3) (layer "F.Cu") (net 4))
 (segment (start 74.8 69) (end 73.9 69.9) (width 0.3) (layer "F.Cu") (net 4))
 (segment (start 92.7 60.4) (end 92.7 60.3) (width 0.3) (layer "F.Cu") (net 7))
 (segment (start 92.8 62.8) (end 92.7 62.7) (width 0.3) (layer "F.Cu") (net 7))
 (segment (start 94 57) (end 100.5 57) (width 0.3) (layer "F.Cu") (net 7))
 (segment (start 93.1 67.2) (end 93.2 67.3) (width 0.3) (layer "F.Cu") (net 7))
 (segment (start 93.2 67.3) (end 93.4 67.3) (width 0.3) (layer "F.Cu") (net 7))
 (segment (start 92.9 60) (end 94 58.9) (width 0.3) (layer "F.Cu") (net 7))
 (segment (start 92.8 67) (end 92.8 62.8) (width 0.3) (layer "F.Cu") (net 7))
 (segment (start 94 58.9) (end 94 57) (width 0.3) (layer "F.Cu") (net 7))
 (segment (start 92.7 62.6) (end 92.6 62.5) (width 0.3) (layer "F.Cu") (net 7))
 (segment (start 92.9 60.1) (end 92.9 60) (width 0.3) (layer "F.Cu") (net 7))
 (segment (start 92.825 67) (end 92.8 67) (width 0.3) (layer "F.Cu") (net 7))
 (segment (start 92.7 60.3) (end 92.9 60.1) (width 0.3) (layer "F.Cu") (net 7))
 (segment (start 93.6 67.4) (end 95.2 69) (width 0.3) (layer "F.Cu") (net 7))
 (segment (start 92.6 60.5) (end 92.7 60.4) (width 0.3) (layer "F.Cu") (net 7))
 (segment (start 92.825 67) (end 92.8 67) (width 0.3) (layer "F.Cu") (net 7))
 (segment (start 93 67.2) (end 93.1 67.2) (width 0.3) (layer "F.Cu") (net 7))
 (segment (start 92.7 62.7) (end 92.7 62.6) (width 0.3) (layer "F.Cu") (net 7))
 (segment (start 93.4 67.3) (end 93.5 67.4) (width 0.3) (layer "F.Cu") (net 7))
 (segment (start 92.8 67) (end 93 67.2) (width 0.3) (layer "F.Cu") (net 7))
 (segment (start 92.6 62.5) (end 92.6 60.5) (width 0.3) (layer "F.Cu") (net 7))
 (segment (start 93.5 67.4) (end 93.6 67.4) (width 0.3) (layer "F.Cu") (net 7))
 (segment (start 95.2 69) (end 95.175 69) (width 0.3) (layer "F.Cu") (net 7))
 (segment (start 95.8 68.1) (end 95.6 67.9) (width 0.3) (layer "F.Cu") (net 5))
 (segment (start 96.825 69) (end 96.8 69) (width 0.3) (layer "F.Cu") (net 5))
 (segment (start 98.9 70.8) (end 98.8 70.7) (width 0.3) (layer "F.Cu") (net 5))
 (segment (start 99.2 71) (end 99 70.8) (width 0.3) (layer "F.Cu") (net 5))
 (segment (start 96.8 69) (end 96.825 69) (width 0.3) (layer "F.Cu") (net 5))
 (segment (start 99 70.8) (end 98.9 70.8) (width 0.3) (layer "F.Cu") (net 5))
 (segment (start 95.6 67.9) (end 95.2 67.9) (width 0.3) (layer "F.Cu") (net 5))
 (segment (start 98.8 70.7) (end 98.6 70.7) (width 0.3) (layer "F.Cu") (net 5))
 (segment (start 98.5 70.6) (end 98.4 70.6) (width 0.3) (layer "F.Cu") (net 5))
 (segment (start 99.225 71) (end 99.2 71) (width 0.3) (layer "F.Cu") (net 5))
 (segment (start 98.6 70.7) (end 98.5 70.6) (width 0.3) (layer "F.Cu") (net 5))
 (segment (start 96.8 69) (end 95.9 68.1) (width 0.3) (layer "F.Cu") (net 5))
 (segment (start 98.4 70.6) (end 96.8 69) (width 0.3) (layer "F.Cu") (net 5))
 (segment (start 95.9 68.1) (end 95.8 68.1) (width 0.3) (layer "F.Cu") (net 5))
 (via (at 95.2 67.9) (size 0.6) (drill 0.3) (layers "F.Cu" "B.Cu") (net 5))
 (segment (start 57 66.599999) (end 57 66.62) (width 0.3) (layer "B.Cu") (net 5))
 (segment (start 93.3 67.9) (end 92.7 67.3) (width 0.3) (layer "B.Cu") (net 5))
 (segment (start 87 67.3) (end 86.6 66.9) (width 0.3) (layer "B.Cu") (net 5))
 (segment (start 86.6 66.9) (end 57.3 66.9) (width 0.3) (layer "B.Cu") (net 5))
 (segment (start 95.2 67.9) (end 93.3 67.9) (width 0.3) (layer "B.Cu") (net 5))
 (segment (start 92.7 67.3) (end 87 67.3) (width 0.3) (layer "B.Cu") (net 5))
 (segment (start 57.3 66.9) (end 57 66.599999) (width 0.3) (layer "B.Cu") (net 5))
 (segment (start 67.5 74) (end 67.6 74) (width 0.3) (layer "F.Cu") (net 6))
 (segment (start 72.3 80.2) (end 74.1 82) (width 0.3) (layer "F.Cu") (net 6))
 (segment (start 58.4 69.6) (end 58.5 69.7) (width 0.3) (layer "F.Cu") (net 6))
 (segment (start 72 78.3) (end 72.1 78.4) (width 0.3) (layer "F.Cu") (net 6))
 (segment (start 71.8 78) (end 71.825 78) (width 0.3) (layer "F.Cu") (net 6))
 (segment (start 57.4 69.5) (end 57.6 69.5) (width 0.3) (layer "F.Cu") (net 6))
 (segment (start 67.7 74.1) (end 67.9 74.1) (width 0.3) (layer "F.Cu") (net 6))
 (segment (start 66.5 73.1) (end 66.599999 73.1) (width 0.3) (layer "F.Cu") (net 6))
 (segment (start 58.5 69.7) (end 63.1 69.7) (width 0.3) (layer "F.Cu") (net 6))
 (segment (start 72.1 78.6) (end 72.2 78.7) (width 0.3) (layer "F.Cu") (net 6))
 (segment (start 66.599999 73.1) (end 67.5 74) (width 0.3) (layer "F.Cu") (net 6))
 (segment (start 71.825 78) (end 71.8 78) (width 0.3) (layer "F.Cu") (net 6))
 (segment (start 57.3 69.4) (end 57.4 69.5) (width 0.3) (layer "F.Cu") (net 6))
 (segment (start 57 69.16) (end 57 69.2) (width 0.3) (layer "F.Cu") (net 6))
 (segment (start 67.6 74) (end 67.7 74.1) (width 0.3) (layer "F.Cu") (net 6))
 (segment (start 72 78.2) (end 72 78.3) (width 0.3) (layer "F.Cu") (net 6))
 (segment (start 72.2 79.4) (end 72.3 79.5) (width 0.3) (layer "F.Cu") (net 6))
 (segment (start 63.1 69.7) (end 66.5 73.1) (width 0.3) (layer "F.Cu") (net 6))
 (segment (start 57.6 69.5) (end 57.7 69.6) (width 0.3) (layer "F.Cu") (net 6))
 (segment (start 57.7 69.6) (end 58.4 69.6) (width 0.3) (layer "F.Cu") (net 6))
 (segment (start 57.2 69.4) (end 57.3 69.4) (width 0.3) (layer "F.Cu") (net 6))
 (segment (start 72.2 78.7) (end 72.2 79.4) (width 0.3) (layer "F.Cu") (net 6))
 (segment (start 67.9 74.1) (end 71.8 78) (width 0.3) (layer "F.Cu") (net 6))
 (segment (start 72.1 78.4) (end 72.1 78.6) (width 0.3) (layer "F.Cu") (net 6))
 (segment (start 57 69.2) (end 57.2 69.4) (width 0.3) (layer "F.Cu") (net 6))
 (segment (start 71.8 78) (end 72 78.2) (width 0.3) (layer "F.Cu") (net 6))
 (segment (start 74.1 82) (end 74.0625 81.95) (width 0.3) (layer "F.Cu") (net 6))
 (segment (start 72.3 79.5) (end 72.3 80.2) (width 0.3) (layer "F.Cu") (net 6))
 (segment (start 97.1 81) (end 94.8 81) (width 0.3) (layer "F.Cu") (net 8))
 (segment (start 94.8 81) (end 94.825 81) (width 0.3) (layer "F.Cu") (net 8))
 (segment (start 97.0625 81) (end 97.1 81) (width 0.3) (layer "F.Cu") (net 8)))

